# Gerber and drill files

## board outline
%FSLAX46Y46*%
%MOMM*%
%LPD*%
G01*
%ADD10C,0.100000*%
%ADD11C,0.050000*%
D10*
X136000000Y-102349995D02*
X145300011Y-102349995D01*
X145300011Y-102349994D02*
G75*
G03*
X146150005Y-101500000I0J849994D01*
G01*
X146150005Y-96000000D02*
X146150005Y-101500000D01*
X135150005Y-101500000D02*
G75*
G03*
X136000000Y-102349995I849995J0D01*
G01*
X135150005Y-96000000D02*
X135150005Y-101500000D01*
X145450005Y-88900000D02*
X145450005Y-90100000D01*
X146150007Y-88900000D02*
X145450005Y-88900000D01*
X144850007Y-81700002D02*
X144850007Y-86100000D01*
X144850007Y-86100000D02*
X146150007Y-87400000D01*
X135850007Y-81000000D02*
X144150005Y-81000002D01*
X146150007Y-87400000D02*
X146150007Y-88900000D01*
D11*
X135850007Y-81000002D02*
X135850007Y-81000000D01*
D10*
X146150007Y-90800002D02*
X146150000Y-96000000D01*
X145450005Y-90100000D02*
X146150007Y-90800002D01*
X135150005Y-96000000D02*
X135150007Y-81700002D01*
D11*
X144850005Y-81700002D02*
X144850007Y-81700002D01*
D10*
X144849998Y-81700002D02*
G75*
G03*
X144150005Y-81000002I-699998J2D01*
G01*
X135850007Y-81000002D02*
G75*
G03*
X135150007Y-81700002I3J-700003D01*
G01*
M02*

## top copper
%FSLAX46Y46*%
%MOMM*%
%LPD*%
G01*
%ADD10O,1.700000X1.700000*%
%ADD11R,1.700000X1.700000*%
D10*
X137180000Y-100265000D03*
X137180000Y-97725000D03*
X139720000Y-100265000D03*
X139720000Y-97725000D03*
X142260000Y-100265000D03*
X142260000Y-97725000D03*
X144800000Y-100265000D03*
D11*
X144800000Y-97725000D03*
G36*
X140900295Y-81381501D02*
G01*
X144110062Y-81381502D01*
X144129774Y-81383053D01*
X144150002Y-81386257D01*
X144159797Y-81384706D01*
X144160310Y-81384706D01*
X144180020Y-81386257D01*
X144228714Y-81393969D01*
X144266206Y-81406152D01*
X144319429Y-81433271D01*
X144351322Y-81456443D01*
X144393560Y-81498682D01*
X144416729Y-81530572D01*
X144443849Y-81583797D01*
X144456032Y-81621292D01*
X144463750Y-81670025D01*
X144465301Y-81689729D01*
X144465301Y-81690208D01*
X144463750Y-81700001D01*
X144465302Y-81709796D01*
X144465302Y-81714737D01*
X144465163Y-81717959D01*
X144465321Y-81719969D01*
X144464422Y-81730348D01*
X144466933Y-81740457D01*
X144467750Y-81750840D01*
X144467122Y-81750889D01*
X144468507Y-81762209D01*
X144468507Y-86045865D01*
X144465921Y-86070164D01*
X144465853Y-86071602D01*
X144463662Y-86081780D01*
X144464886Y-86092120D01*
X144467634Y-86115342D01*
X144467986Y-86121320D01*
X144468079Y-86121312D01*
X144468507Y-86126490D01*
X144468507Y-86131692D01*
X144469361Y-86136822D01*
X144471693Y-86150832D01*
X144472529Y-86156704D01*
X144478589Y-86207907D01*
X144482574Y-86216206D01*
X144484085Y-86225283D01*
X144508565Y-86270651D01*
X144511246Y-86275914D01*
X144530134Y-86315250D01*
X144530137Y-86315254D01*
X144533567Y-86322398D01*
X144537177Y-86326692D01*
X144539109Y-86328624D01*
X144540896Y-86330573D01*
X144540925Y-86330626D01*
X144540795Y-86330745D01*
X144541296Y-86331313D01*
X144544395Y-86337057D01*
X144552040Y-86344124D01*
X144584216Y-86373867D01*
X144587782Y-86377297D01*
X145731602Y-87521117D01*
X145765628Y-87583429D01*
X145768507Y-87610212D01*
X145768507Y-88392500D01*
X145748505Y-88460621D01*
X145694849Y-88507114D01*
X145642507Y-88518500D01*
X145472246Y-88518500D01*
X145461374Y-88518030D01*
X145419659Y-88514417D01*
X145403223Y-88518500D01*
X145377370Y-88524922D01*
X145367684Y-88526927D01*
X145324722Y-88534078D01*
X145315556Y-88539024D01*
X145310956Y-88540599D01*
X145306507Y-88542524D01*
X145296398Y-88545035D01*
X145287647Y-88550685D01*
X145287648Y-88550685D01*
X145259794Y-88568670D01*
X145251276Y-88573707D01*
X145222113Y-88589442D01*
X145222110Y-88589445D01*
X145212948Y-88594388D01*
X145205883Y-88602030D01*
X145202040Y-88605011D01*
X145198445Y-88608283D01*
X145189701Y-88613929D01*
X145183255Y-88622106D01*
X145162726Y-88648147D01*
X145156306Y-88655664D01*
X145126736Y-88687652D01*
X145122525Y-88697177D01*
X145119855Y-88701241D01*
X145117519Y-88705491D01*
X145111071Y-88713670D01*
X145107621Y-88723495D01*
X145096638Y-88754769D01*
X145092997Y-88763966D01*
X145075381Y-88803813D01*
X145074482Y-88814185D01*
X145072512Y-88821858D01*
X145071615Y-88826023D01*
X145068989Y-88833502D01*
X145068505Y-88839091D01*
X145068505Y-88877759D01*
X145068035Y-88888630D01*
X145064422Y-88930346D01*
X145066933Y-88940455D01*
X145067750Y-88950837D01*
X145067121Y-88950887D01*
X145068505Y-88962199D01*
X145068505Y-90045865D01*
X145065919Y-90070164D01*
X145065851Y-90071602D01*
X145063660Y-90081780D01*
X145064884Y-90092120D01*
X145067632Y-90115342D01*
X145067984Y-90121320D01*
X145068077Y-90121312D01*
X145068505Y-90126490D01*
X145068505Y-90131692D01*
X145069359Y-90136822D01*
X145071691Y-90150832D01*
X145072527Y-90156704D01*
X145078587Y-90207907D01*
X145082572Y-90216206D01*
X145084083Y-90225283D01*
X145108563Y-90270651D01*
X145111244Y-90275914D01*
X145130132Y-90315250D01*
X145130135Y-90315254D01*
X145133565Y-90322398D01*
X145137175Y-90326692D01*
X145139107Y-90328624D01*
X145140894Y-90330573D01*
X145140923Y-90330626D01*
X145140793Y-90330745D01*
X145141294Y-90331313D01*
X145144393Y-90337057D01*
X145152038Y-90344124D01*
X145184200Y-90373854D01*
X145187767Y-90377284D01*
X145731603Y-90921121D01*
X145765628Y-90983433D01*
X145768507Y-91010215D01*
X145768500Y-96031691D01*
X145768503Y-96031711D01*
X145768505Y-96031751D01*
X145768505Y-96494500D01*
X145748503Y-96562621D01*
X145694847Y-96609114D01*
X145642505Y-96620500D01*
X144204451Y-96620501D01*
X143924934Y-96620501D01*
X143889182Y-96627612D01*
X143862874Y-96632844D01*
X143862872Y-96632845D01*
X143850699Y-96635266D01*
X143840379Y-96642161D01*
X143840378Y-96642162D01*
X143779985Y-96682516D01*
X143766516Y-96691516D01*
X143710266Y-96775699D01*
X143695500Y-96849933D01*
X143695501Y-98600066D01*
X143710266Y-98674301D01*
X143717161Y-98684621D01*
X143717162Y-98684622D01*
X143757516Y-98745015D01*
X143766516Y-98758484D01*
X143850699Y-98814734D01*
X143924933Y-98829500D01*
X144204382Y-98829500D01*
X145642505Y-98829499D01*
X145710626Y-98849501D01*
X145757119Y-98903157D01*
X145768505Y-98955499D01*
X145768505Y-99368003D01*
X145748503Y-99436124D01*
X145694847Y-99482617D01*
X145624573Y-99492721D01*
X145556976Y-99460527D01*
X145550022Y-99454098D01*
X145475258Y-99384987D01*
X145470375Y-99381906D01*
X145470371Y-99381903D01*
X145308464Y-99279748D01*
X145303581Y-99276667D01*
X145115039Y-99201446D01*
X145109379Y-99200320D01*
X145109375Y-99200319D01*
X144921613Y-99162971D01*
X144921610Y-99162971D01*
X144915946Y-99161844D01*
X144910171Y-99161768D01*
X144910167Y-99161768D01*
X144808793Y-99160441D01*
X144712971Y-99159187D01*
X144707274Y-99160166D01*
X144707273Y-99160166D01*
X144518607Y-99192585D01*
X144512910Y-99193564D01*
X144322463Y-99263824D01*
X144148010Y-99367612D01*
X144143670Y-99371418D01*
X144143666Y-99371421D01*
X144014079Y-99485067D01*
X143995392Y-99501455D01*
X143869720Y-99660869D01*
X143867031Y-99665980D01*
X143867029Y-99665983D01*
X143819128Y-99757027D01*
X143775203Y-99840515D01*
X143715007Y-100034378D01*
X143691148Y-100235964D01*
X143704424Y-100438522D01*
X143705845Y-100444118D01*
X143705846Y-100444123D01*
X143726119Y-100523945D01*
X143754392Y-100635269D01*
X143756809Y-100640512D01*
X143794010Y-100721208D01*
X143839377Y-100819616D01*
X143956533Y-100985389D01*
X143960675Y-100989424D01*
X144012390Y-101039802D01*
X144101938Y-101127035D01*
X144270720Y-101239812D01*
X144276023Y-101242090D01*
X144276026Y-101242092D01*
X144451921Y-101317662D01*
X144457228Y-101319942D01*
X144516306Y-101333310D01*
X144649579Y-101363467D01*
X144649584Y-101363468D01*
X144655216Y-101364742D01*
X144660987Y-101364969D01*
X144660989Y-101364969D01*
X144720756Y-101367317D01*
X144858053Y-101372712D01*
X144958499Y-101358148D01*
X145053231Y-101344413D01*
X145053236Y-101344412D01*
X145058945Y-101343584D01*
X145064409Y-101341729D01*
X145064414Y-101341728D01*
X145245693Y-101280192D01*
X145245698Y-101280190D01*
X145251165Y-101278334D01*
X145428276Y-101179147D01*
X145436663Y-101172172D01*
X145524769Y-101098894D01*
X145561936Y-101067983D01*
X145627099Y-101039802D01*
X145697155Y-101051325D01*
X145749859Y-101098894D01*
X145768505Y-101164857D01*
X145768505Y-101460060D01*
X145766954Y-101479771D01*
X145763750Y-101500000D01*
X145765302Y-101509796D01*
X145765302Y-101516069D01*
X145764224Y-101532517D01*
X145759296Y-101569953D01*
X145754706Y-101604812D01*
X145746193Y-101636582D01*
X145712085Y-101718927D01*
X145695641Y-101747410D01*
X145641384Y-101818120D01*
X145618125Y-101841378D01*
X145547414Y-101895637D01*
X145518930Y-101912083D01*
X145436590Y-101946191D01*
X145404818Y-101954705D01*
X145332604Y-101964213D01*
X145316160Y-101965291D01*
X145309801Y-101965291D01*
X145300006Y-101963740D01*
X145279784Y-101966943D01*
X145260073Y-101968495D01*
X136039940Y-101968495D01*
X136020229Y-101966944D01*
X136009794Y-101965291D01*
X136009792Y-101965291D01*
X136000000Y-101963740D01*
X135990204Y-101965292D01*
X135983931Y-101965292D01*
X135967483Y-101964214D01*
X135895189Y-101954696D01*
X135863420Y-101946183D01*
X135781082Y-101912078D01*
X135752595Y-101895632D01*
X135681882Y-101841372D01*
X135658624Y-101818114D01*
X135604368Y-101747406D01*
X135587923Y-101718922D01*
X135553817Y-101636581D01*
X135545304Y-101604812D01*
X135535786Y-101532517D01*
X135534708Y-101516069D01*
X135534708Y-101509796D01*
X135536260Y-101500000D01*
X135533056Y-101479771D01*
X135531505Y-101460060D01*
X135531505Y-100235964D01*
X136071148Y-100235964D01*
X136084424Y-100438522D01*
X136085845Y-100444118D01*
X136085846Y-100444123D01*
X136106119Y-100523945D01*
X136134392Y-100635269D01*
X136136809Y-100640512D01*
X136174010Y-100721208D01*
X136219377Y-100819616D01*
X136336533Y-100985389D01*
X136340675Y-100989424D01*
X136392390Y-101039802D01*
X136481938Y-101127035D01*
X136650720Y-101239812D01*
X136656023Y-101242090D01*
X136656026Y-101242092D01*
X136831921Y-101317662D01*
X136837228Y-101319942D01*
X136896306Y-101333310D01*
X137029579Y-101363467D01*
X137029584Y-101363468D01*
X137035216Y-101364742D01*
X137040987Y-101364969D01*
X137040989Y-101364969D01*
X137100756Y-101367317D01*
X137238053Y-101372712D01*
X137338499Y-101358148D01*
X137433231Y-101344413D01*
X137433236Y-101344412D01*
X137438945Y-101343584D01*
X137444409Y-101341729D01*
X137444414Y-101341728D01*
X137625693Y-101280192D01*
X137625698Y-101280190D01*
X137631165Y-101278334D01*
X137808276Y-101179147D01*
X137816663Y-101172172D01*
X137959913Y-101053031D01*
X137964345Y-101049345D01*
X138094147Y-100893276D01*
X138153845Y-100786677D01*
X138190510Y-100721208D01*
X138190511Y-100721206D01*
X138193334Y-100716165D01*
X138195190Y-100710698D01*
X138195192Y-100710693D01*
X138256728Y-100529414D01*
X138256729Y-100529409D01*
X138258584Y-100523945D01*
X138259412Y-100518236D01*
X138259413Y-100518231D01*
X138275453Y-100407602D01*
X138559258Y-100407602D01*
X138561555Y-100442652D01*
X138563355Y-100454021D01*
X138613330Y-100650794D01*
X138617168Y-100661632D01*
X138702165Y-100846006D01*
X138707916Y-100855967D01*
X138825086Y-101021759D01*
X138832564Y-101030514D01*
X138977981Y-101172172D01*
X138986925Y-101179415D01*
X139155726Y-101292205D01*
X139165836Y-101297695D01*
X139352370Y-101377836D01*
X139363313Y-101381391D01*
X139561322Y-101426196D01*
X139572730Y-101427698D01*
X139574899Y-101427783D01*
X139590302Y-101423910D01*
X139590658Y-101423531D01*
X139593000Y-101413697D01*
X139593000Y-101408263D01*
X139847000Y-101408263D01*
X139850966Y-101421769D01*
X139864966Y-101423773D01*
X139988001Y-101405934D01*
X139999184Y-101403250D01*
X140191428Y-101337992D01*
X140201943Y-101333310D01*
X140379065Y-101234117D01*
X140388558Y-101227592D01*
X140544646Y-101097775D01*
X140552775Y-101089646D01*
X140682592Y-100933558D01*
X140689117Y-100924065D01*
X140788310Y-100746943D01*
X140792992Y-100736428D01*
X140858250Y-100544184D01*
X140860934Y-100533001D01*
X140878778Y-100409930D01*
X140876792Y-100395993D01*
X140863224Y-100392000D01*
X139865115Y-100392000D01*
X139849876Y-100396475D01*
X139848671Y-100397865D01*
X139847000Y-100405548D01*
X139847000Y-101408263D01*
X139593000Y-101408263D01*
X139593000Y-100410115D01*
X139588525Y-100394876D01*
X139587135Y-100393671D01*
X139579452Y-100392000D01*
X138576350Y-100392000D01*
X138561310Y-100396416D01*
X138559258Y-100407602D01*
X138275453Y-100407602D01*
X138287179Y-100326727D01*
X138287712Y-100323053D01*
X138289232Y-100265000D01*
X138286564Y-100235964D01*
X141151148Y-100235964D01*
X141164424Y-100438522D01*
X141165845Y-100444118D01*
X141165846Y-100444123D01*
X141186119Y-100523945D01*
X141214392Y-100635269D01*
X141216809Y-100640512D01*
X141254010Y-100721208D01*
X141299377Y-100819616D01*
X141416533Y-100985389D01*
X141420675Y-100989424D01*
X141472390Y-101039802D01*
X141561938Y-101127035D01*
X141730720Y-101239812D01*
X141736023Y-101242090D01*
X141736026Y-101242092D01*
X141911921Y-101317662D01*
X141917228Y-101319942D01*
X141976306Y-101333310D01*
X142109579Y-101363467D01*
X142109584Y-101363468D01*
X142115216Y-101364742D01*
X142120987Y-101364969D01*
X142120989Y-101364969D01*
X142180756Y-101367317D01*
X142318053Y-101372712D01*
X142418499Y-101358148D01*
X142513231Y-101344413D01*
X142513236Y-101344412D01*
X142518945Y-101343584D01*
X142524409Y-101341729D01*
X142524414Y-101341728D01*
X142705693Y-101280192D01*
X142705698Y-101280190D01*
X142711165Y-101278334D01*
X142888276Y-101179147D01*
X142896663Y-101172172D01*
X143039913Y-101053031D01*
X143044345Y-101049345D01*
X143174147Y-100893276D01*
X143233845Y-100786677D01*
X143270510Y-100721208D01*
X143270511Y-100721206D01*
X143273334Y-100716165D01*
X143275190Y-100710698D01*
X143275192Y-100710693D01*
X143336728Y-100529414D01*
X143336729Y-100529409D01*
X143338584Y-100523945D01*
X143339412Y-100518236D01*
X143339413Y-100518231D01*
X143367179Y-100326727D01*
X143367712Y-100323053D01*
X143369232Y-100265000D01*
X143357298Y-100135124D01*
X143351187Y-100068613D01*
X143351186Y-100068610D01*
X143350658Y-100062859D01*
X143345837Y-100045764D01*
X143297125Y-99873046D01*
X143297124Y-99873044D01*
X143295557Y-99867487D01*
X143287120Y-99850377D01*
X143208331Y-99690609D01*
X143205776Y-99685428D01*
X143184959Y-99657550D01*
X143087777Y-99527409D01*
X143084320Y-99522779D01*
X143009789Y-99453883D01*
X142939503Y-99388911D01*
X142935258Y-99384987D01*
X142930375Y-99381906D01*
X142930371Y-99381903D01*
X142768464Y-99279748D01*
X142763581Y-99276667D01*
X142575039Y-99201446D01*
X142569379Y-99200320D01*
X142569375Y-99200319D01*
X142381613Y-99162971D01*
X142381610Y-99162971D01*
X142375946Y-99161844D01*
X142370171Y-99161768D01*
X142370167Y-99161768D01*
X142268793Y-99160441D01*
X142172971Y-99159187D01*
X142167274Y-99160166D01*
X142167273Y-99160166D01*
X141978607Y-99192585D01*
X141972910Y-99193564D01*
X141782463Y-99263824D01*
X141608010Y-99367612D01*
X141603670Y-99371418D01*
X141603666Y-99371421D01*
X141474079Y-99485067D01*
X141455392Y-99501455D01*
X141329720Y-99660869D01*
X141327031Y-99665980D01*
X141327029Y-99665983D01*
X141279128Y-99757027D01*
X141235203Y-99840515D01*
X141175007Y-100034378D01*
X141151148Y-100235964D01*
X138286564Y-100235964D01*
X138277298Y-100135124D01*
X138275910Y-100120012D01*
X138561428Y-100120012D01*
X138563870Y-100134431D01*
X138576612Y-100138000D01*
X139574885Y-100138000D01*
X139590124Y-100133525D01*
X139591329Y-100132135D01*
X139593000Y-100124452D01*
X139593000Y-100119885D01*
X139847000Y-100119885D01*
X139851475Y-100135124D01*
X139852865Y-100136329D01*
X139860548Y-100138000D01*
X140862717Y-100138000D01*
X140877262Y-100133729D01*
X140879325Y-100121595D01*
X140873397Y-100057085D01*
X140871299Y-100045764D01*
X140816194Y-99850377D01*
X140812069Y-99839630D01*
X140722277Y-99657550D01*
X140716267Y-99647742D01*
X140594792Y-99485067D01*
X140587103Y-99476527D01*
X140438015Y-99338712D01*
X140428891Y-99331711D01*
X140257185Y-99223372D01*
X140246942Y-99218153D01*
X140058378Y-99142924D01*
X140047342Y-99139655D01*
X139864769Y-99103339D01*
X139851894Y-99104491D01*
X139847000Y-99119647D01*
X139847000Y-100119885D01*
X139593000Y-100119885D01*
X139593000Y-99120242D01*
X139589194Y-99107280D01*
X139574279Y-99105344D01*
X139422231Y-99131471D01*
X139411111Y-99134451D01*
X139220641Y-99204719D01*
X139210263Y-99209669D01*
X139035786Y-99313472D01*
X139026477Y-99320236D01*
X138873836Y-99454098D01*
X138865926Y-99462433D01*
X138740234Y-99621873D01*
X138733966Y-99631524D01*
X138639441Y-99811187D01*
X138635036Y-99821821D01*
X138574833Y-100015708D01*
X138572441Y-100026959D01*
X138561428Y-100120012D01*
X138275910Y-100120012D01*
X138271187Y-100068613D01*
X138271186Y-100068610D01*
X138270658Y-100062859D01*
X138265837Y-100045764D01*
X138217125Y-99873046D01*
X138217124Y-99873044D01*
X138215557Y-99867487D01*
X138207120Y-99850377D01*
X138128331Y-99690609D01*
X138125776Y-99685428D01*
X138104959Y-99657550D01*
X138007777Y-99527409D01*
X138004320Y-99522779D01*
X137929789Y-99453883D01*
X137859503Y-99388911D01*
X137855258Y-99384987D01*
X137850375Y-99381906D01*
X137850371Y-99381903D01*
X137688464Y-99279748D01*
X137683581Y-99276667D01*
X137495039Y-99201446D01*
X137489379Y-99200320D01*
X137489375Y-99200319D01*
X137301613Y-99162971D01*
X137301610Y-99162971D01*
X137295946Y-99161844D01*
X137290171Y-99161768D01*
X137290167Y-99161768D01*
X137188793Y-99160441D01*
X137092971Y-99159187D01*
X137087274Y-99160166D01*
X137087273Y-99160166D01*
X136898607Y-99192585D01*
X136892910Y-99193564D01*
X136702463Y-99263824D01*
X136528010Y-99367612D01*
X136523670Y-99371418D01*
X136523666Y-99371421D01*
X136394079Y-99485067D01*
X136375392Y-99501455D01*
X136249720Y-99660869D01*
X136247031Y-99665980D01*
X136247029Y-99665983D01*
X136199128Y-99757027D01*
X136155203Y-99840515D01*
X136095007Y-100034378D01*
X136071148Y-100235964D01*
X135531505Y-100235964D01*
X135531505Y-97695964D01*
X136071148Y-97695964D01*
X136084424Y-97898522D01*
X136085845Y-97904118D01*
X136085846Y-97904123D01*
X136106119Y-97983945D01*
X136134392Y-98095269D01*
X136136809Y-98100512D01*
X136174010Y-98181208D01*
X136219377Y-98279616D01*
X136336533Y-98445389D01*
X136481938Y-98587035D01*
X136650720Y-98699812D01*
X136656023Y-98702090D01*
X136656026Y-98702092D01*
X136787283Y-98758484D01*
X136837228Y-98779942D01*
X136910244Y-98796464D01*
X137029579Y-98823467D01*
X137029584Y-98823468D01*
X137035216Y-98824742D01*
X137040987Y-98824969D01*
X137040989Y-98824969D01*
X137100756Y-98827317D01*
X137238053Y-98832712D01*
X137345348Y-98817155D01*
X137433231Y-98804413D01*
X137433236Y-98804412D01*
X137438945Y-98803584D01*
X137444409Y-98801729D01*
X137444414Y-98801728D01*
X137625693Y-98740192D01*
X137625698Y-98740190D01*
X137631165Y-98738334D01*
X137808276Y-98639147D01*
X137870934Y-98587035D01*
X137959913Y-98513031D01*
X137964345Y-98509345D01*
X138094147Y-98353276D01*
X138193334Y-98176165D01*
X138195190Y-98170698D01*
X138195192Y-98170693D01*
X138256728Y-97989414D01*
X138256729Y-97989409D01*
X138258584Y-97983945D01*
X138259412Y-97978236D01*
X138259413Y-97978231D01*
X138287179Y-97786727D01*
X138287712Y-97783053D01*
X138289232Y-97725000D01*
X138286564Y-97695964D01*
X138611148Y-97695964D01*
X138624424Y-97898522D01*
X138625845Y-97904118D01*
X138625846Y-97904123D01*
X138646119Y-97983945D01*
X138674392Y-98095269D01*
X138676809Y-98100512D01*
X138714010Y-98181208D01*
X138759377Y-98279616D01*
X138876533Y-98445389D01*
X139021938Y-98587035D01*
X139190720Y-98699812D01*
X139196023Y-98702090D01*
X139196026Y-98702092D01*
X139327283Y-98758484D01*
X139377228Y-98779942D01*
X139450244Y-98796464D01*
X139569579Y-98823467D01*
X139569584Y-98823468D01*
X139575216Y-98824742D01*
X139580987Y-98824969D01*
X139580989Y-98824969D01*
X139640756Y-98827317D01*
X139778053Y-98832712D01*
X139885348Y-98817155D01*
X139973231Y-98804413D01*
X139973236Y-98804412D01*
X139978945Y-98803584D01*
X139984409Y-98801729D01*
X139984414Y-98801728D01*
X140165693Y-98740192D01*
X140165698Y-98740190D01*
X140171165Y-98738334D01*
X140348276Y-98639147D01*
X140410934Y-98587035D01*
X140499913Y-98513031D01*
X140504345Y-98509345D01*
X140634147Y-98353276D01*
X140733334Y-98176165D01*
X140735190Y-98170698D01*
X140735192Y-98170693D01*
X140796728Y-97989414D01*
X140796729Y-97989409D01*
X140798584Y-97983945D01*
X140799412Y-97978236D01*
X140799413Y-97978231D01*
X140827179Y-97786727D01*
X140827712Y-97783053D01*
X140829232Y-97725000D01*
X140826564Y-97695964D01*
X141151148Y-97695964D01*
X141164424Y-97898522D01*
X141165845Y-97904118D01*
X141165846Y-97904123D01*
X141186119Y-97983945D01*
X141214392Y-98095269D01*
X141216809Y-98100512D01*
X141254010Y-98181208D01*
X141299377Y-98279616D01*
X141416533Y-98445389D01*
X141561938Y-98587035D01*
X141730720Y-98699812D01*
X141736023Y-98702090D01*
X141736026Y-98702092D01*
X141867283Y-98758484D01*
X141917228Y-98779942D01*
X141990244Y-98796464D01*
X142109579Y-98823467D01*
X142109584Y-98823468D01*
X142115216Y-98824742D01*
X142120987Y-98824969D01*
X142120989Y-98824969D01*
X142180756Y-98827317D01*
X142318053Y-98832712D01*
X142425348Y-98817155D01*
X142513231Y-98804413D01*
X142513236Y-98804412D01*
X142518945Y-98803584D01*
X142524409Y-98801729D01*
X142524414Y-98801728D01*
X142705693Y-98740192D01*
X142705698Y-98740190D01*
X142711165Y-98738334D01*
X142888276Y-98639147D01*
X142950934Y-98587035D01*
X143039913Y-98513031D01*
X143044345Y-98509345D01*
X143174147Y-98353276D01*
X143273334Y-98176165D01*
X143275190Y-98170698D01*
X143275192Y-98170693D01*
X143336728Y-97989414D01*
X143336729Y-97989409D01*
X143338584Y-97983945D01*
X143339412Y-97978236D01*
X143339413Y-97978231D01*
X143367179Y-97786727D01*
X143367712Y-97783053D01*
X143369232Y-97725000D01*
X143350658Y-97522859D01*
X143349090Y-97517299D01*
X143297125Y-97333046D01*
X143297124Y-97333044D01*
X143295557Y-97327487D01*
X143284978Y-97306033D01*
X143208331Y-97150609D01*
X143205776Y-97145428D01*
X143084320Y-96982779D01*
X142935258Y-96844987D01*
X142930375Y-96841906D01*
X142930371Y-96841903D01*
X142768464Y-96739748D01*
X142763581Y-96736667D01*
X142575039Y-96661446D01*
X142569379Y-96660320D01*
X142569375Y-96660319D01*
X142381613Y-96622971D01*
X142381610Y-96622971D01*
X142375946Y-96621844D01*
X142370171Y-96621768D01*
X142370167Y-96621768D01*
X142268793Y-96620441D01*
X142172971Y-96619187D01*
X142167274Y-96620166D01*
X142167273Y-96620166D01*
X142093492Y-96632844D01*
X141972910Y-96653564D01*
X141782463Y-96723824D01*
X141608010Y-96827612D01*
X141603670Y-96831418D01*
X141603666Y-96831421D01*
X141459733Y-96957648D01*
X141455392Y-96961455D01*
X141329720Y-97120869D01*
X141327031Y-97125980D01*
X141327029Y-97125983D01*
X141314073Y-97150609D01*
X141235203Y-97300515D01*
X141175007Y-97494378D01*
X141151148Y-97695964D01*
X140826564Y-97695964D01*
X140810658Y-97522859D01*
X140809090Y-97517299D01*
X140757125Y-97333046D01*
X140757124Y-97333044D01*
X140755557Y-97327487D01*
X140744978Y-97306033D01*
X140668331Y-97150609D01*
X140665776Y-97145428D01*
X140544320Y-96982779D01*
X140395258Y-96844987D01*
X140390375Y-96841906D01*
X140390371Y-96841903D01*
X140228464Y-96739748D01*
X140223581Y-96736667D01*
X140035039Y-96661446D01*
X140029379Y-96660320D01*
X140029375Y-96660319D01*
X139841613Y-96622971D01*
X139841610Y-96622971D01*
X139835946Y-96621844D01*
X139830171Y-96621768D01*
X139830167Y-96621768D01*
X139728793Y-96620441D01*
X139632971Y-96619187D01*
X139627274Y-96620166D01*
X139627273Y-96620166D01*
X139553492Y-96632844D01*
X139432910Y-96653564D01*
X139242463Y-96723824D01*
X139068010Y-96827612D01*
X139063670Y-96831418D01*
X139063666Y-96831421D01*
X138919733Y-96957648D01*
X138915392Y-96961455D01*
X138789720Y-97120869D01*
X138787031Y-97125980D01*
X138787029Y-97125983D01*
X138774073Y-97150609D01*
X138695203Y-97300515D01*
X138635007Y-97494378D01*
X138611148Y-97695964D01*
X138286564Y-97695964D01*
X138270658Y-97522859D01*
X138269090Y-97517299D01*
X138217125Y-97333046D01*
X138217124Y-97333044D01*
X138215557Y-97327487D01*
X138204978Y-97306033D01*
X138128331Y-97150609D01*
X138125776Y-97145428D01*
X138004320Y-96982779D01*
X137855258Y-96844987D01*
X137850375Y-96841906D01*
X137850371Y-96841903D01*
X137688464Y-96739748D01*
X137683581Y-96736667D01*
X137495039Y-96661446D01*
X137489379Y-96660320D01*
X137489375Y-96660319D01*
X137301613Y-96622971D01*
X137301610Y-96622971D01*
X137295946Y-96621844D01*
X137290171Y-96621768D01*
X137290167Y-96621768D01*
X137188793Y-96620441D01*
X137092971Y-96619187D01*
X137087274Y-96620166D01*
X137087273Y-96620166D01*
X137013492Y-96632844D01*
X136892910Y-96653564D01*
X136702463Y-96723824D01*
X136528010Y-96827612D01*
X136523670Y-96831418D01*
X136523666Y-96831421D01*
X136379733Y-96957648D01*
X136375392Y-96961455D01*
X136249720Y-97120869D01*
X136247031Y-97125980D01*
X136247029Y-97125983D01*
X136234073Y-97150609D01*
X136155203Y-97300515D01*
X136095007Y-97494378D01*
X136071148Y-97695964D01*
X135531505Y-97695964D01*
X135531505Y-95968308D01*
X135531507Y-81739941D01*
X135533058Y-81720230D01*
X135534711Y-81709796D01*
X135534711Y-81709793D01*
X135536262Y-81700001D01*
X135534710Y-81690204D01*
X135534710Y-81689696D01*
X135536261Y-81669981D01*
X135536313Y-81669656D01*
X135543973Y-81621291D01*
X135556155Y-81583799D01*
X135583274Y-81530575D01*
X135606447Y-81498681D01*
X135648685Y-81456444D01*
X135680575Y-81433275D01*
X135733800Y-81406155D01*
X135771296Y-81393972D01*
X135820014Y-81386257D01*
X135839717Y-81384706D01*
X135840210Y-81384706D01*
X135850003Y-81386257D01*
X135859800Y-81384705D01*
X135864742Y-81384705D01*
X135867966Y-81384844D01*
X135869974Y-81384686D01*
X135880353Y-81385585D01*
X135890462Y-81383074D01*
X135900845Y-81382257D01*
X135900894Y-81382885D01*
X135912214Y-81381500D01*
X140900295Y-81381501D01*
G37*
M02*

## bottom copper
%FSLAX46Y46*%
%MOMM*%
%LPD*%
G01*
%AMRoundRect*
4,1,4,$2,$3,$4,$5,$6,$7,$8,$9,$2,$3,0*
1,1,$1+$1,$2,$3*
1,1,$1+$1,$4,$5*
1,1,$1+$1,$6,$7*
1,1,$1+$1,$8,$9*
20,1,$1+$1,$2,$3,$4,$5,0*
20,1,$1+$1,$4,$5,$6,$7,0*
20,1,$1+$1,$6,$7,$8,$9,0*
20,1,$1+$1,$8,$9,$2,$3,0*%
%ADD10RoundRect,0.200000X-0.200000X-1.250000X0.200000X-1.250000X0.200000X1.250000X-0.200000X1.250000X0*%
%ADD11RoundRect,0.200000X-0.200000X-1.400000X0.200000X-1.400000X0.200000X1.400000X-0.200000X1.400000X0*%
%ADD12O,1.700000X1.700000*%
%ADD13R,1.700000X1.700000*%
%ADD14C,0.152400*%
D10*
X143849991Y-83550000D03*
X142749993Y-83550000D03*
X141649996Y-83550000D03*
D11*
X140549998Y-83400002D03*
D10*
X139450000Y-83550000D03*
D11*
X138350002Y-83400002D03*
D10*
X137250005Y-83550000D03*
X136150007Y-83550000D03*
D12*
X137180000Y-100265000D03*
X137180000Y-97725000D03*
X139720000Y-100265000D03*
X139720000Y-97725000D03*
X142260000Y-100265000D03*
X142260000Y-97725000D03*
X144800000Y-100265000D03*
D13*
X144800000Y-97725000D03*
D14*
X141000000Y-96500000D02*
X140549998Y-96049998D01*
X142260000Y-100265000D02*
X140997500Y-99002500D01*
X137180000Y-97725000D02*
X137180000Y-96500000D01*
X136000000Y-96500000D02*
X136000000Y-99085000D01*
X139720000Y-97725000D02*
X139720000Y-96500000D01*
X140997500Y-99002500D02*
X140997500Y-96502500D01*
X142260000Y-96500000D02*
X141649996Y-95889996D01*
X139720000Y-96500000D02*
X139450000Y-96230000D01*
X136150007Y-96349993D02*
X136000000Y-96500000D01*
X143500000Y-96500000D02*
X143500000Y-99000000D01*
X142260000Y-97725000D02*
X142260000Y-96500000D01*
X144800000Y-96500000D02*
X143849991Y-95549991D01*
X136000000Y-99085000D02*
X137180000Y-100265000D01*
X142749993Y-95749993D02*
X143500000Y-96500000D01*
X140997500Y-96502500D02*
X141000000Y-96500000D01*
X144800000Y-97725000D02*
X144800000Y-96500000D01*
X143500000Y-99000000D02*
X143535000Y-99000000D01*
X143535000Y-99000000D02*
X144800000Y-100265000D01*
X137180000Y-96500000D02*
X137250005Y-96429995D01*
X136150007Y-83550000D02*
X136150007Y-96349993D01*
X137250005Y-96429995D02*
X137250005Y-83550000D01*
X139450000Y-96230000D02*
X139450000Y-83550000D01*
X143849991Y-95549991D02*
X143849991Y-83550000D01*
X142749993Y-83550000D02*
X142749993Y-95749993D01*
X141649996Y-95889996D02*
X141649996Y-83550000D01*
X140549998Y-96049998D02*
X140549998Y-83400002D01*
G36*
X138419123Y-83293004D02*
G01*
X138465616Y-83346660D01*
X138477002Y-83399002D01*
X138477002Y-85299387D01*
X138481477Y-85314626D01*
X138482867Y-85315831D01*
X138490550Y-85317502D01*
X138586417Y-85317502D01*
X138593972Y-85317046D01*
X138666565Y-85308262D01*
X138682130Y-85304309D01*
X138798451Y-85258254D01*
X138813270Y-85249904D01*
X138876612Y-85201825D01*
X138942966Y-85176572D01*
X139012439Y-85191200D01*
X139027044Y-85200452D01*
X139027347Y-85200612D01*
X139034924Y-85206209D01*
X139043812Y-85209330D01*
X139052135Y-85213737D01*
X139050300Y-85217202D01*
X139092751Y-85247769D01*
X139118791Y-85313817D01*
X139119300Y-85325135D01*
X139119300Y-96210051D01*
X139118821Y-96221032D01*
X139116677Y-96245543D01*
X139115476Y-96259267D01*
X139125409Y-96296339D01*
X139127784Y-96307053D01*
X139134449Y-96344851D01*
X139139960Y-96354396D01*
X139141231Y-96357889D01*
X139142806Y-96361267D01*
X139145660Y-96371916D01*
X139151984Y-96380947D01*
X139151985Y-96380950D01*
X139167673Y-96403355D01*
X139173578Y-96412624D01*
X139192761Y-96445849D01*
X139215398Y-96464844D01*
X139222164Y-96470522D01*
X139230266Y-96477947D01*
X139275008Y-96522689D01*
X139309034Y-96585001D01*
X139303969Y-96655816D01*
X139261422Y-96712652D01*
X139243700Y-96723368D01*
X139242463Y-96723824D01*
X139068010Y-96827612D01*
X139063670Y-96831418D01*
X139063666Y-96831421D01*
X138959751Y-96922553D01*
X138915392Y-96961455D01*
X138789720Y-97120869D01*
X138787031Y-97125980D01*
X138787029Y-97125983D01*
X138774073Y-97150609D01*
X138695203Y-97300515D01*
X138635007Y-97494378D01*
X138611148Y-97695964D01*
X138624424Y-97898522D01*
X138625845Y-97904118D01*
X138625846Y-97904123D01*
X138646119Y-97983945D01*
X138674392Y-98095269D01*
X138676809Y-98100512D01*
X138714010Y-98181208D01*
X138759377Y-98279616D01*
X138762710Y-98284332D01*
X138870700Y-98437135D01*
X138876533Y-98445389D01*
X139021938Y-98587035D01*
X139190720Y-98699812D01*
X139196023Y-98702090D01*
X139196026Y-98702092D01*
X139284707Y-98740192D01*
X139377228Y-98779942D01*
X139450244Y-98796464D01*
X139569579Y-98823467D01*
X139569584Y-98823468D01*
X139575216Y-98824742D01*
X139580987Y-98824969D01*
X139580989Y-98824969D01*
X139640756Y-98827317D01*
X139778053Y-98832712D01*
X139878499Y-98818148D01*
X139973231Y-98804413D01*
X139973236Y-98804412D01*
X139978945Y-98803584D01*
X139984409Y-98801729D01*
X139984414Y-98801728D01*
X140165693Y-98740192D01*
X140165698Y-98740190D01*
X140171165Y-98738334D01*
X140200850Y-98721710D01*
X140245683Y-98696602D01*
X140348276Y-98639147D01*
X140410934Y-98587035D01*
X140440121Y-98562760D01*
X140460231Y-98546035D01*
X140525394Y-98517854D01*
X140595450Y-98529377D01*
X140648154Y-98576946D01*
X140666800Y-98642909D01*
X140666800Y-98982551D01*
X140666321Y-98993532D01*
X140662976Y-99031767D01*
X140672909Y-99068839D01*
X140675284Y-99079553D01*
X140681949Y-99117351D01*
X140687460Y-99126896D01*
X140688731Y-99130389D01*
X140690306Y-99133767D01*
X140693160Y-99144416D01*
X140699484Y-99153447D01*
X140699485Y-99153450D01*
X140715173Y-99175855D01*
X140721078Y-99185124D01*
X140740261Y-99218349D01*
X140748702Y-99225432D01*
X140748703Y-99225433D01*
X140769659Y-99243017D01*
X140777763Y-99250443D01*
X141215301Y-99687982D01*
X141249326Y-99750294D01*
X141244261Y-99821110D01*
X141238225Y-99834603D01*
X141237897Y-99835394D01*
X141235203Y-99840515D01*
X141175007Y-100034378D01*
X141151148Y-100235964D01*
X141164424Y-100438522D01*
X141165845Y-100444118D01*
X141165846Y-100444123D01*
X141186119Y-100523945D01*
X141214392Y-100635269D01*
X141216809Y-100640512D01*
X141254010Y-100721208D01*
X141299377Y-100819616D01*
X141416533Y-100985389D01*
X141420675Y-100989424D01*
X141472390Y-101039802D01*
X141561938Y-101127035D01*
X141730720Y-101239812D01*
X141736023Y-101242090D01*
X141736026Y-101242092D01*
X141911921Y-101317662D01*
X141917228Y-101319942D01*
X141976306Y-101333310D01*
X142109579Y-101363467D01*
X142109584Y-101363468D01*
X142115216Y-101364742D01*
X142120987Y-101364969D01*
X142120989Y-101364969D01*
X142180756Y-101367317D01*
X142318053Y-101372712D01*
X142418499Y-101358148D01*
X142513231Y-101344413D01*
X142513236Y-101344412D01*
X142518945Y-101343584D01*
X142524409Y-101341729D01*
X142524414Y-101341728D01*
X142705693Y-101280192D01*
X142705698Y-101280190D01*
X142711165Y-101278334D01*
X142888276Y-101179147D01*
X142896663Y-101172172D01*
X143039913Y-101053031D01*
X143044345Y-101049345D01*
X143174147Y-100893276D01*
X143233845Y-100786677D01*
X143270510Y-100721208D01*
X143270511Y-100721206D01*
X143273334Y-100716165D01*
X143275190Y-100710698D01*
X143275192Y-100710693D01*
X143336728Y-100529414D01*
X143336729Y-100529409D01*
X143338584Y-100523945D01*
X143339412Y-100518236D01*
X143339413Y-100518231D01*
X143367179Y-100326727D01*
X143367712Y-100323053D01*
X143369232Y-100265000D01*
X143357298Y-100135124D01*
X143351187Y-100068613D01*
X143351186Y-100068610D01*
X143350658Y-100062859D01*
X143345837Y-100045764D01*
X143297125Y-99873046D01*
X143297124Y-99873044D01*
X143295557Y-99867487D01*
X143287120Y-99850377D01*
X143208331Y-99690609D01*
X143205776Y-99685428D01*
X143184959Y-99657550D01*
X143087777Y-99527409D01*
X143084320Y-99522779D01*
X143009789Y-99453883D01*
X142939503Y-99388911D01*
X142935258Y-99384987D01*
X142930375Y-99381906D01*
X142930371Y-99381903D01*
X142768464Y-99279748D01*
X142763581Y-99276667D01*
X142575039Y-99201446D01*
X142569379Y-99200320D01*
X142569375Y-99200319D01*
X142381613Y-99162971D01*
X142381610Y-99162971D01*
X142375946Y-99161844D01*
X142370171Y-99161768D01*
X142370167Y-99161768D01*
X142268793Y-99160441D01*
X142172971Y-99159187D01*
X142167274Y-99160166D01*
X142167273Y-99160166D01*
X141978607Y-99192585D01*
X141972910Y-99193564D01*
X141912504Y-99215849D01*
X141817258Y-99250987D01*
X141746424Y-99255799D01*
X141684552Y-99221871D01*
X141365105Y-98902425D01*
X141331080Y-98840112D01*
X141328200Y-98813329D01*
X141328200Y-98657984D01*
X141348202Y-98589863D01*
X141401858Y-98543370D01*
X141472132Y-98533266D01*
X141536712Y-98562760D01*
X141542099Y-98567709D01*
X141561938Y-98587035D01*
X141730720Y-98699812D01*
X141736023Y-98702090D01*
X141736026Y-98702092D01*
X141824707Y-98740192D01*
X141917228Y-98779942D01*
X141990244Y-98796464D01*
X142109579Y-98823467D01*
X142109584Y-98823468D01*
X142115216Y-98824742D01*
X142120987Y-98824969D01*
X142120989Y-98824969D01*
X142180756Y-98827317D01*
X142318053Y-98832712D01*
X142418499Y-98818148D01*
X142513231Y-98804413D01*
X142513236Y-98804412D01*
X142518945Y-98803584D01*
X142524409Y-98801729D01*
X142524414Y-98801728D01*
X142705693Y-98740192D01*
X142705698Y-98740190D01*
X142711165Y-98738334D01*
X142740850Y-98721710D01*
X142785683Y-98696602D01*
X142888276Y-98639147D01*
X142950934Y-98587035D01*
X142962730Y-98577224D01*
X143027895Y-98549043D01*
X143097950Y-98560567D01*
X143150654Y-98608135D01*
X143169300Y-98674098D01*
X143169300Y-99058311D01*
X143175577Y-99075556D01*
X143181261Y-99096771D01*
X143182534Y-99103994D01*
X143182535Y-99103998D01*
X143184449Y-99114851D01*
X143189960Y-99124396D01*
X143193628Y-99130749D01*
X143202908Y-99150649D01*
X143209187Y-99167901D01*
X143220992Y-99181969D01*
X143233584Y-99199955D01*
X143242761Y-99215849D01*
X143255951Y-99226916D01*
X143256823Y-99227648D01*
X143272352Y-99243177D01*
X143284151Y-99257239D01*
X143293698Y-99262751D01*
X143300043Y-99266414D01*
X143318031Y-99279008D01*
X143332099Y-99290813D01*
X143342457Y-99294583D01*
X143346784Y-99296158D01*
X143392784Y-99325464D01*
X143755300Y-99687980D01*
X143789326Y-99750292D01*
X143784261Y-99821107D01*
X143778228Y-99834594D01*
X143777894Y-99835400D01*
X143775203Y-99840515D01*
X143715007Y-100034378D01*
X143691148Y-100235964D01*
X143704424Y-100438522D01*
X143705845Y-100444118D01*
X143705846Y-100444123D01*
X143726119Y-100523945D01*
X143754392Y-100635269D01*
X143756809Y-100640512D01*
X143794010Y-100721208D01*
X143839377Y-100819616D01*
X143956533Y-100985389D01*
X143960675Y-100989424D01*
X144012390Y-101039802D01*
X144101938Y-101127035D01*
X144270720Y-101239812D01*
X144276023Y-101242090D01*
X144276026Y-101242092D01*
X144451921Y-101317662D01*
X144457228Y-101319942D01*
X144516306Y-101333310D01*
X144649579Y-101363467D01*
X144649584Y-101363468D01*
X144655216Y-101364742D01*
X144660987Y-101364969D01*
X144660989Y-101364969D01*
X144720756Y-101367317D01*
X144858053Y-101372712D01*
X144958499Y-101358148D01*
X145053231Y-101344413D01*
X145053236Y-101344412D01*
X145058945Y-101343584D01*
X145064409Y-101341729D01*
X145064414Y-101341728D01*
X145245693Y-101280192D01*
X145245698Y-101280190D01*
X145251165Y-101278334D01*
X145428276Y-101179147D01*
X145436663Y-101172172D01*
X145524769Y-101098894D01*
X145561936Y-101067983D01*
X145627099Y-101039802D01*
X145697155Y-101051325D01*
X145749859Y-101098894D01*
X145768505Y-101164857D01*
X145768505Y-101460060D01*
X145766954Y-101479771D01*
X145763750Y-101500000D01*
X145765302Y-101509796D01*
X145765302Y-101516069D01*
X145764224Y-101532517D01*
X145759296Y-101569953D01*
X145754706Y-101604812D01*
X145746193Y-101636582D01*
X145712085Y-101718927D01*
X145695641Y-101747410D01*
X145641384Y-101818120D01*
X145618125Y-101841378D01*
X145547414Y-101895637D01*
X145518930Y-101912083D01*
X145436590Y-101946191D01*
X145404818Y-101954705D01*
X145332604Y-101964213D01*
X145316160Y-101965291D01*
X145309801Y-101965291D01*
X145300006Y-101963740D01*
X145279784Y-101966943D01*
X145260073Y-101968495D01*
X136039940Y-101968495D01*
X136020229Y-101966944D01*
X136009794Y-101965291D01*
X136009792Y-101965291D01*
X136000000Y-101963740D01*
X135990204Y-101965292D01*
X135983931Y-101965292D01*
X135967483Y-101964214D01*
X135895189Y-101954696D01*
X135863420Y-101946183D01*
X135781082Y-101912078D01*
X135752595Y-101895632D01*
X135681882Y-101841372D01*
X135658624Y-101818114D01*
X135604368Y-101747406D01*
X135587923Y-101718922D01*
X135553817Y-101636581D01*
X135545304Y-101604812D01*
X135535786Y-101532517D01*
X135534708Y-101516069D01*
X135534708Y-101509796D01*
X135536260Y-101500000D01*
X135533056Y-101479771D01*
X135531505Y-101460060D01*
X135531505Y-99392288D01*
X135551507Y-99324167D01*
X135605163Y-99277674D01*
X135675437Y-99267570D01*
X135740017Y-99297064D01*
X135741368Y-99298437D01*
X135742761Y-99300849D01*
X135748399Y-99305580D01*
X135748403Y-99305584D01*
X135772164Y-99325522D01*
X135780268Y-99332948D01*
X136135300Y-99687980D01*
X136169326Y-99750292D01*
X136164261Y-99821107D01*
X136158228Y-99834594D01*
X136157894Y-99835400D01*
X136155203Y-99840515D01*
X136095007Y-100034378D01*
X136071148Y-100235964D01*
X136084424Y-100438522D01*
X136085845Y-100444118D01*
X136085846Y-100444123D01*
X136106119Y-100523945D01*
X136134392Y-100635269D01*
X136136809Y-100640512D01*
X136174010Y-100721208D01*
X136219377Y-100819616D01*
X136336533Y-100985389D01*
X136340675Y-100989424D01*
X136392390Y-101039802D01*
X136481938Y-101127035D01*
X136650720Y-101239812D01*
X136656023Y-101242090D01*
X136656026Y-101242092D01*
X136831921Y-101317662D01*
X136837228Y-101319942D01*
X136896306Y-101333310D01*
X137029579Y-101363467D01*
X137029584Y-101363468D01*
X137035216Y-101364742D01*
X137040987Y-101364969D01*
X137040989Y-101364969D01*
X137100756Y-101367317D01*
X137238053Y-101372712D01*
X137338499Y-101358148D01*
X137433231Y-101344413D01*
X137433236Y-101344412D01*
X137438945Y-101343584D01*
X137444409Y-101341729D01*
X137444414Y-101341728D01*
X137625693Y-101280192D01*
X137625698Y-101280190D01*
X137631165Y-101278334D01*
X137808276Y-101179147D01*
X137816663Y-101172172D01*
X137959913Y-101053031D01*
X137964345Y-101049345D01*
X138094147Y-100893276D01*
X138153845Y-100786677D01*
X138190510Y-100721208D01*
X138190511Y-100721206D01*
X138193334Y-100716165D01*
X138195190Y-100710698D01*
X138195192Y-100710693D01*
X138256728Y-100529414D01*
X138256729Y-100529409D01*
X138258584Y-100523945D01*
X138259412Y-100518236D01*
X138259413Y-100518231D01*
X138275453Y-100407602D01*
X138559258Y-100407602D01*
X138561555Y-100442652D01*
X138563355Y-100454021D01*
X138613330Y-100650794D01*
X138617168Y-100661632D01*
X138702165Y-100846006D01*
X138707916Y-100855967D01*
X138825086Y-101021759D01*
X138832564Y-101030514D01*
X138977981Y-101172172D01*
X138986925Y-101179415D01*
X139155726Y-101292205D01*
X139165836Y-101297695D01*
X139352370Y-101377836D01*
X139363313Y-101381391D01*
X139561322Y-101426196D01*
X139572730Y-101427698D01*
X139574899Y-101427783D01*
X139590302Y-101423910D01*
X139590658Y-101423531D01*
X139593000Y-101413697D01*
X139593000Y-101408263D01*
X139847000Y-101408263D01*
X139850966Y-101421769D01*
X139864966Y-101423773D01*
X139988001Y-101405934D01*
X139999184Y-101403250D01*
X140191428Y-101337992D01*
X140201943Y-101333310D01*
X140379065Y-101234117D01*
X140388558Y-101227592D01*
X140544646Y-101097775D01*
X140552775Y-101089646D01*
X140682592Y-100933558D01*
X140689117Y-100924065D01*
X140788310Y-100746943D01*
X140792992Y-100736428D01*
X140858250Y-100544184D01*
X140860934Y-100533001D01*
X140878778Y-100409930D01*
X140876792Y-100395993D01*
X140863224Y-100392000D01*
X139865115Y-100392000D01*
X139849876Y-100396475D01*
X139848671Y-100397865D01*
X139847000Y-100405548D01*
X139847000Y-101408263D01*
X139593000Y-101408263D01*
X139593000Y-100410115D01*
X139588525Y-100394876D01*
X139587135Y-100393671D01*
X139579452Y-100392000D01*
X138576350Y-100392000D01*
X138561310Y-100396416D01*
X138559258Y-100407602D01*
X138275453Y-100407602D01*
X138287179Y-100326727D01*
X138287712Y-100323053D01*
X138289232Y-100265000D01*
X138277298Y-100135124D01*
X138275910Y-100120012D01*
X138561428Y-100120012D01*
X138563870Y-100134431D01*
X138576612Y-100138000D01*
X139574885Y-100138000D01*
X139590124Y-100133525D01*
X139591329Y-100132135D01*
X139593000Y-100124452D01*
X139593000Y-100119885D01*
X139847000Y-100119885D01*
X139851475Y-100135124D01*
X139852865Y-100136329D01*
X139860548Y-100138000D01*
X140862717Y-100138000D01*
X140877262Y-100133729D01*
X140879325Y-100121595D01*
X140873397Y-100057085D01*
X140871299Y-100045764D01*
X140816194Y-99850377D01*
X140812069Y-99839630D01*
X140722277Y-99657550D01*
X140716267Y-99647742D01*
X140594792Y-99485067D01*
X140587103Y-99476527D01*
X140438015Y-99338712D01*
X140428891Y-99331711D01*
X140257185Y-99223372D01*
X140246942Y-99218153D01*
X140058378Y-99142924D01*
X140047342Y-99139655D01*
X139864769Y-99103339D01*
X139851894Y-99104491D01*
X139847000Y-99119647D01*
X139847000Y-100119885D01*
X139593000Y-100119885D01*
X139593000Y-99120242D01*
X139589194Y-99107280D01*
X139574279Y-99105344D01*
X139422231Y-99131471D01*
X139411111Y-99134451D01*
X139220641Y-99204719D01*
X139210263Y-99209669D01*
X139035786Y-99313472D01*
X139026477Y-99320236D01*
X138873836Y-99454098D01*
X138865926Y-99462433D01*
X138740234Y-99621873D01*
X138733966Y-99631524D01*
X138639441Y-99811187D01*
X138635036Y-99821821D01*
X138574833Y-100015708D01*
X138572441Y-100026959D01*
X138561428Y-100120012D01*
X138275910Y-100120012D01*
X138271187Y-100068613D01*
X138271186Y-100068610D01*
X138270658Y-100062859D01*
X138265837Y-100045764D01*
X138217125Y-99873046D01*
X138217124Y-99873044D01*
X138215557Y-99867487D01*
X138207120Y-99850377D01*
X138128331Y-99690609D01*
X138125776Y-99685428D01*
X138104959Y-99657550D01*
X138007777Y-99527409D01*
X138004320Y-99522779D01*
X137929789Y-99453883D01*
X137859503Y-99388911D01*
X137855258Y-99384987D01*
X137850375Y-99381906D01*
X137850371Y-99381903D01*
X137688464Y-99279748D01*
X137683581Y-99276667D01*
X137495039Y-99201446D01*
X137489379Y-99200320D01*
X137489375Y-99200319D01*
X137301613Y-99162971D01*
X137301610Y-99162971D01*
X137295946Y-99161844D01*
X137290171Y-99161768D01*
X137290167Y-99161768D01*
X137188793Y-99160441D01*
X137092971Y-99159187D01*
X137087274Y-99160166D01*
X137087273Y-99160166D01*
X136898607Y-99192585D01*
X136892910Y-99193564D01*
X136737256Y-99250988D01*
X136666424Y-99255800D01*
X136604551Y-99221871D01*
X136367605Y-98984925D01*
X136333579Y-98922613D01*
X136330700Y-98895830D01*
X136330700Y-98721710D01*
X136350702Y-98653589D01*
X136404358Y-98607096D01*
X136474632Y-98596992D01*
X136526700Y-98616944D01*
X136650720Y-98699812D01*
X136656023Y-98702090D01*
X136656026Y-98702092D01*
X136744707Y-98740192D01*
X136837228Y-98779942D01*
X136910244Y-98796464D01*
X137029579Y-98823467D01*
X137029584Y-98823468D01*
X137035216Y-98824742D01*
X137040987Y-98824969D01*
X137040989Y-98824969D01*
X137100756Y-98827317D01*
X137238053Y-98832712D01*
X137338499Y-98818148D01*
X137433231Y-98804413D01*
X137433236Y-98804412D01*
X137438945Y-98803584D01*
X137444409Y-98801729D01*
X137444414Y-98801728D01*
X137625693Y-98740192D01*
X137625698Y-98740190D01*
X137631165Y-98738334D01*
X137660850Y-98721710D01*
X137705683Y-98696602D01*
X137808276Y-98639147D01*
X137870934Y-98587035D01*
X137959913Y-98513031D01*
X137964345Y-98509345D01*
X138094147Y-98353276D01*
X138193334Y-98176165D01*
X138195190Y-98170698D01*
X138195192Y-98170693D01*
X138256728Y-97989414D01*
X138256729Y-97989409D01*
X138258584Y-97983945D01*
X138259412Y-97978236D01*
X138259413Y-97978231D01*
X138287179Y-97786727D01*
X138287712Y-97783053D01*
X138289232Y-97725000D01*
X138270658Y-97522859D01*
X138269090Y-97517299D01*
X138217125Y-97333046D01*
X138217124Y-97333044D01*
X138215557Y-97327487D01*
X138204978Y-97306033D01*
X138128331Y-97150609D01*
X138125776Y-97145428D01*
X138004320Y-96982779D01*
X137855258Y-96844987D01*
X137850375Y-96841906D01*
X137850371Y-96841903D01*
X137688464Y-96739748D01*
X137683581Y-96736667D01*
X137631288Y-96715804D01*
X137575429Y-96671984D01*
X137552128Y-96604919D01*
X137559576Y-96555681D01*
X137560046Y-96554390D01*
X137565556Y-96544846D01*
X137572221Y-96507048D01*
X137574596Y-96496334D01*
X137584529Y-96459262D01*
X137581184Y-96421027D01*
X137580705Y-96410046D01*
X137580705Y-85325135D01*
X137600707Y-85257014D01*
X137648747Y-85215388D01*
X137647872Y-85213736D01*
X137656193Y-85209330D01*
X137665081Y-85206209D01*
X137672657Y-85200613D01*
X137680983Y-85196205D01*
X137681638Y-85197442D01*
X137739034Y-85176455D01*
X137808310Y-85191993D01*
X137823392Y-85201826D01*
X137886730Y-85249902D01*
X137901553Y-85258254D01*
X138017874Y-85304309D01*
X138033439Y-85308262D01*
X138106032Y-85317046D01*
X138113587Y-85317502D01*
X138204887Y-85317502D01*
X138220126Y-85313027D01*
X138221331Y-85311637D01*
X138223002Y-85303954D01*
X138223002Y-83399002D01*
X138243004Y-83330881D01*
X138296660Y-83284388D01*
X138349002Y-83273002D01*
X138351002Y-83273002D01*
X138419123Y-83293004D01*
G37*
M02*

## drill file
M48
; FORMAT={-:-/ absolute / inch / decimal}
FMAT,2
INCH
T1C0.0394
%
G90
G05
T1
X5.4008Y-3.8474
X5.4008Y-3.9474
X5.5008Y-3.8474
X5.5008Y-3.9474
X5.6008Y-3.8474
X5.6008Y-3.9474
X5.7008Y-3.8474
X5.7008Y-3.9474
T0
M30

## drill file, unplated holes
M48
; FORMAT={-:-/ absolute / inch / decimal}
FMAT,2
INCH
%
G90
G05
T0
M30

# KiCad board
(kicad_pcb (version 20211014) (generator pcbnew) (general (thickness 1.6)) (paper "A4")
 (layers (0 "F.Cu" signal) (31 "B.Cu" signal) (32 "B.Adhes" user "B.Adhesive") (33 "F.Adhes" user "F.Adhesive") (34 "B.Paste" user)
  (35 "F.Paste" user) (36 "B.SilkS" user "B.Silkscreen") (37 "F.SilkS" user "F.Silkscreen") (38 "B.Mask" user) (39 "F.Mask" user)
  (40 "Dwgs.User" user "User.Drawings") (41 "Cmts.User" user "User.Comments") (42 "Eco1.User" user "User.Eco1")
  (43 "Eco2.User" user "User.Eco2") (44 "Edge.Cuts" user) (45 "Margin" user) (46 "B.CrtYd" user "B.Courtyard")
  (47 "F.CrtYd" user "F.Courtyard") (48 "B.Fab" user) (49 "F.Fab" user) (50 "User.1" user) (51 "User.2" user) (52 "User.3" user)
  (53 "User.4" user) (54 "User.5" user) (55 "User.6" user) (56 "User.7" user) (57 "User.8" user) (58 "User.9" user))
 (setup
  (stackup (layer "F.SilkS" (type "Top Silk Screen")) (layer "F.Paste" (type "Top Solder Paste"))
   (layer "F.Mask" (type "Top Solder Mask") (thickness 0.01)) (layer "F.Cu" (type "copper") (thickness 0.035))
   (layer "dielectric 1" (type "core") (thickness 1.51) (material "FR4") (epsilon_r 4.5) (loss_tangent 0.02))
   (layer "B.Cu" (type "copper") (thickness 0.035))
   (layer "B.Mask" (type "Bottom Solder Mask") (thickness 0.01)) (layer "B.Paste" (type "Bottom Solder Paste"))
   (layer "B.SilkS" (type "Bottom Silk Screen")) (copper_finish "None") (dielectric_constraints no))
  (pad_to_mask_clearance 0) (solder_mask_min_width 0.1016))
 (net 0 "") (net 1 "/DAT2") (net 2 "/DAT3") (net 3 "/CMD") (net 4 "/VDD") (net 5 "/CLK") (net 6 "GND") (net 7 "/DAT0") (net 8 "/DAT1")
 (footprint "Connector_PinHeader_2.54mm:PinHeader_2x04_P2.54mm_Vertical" (layer "F.Cu") (at 144.8 97.725 -90)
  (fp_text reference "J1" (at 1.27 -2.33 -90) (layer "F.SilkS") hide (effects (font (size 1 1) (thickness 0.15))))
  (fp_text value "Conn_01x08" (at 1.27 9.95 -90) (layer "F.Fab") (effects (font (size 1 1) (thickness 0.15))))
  (pad "1" thru_hole rect (at 0 0 270) (size 1.7 1.7) (drill 1) (layers *.Cu *.Mask) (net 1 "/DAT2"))
  (pad "2" thru_hole oval (at 2.54 0 270) (size 1.7 1.7) (drill 1) (layers *.Cu *.Mask) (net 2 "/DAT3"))
  (pad "3" thru_hole oval (at 0 2.54 270) (size 1.7 1.7) (drill 1) (layers *.Cu *.Mask) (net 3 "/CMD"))
  (pad "4" thru_hole oval (at 2.54 2.54 270) (size 1.7 1.7) (drill 1) (layers *.Cu *.Mask) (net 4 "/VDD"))
  (pad "5" thru_hole oval (at 0 5.08 270) (size 1.7 1.7) (drill 1) (layers *.Cu *.Mask) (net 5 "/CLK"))
  (pad "6" thru_hole oval (at 2.54 5.08 270) (size 1.7 1.7) (drill 1) (layers *.Cu *.Mask) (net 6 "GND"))
  (pad "7" thru_hole oval (at 0 7.62 270) (size 1.7 1.7) (drill 1) (layers *.Cu *.Mask) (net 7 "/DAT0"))
  (pad "8" thru_hole oval (at 2.54 7.62 270) (size 1.7 1.7) (drill 1) (layers *.Cu *.Mask) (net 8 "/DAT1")))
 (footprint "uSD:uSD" (layer "F.Cu") (at 140 90)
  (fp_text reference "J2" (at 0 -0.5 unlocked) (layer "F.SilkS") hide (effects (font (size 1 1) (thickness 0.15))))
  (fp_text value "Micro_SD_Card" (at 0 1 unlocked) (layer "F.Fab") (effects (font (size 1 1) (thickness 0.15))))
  (fp_line (start 4.850007 -8.299998) (end 4.850007 -3.9) (layer "Edge.Cuts") (width 0.1))
  (fp_line (start -4.149993 -9) (end 4.150005 -8.999998) (layer "Edge.Cuts") (width 0.1))
  (fp_line (start 4.850005 -8.299998) (end 4.850007 -8.299998) (layer "Edge.Cuts") (width 0.05))
  (fp_line (start 4.850007 -3.9) (end 6.150007 -2.6) (layer "Edge.Cuts") (width 0.1))
  (fp_line (start 6.150007 0.800002) (end 6.15 6) (layer "Edge.Cuts") (width 0.1))
  (fp_line (start 6.150007 -1.1) (end 5.450005 -1.1) (layer "Edge.Cuts") (width 0.1))
  (fp_line (start 5.450005 0.1) (end 6.150007 0.800002) (layer "Edge.Cuts") (width 0.1))
  (fp_line (start 6.150007 -2.6) (end 6.150007 -1.1) (layer "Edge.Cuts") (width 0.1))
  (fp_line (start -4.149993 -8.999998) (end -4.149993 -9) (layer "Edge.Cuts") (width 0.05))
  (fp_line (start -4.849995 6) (end -4.849993 -8.299998) (layer "Edge.Cuts") (width 0.1))
  (fp_line (start 5.450005 -1.1) (end 5.450005 0.1) (layer "Edge.Cuts") (width 0.1))
  (fp_arc (start -4.849993 -8.299998) (mid -4.644967 -8.794972) (end -4.149993 -8.999998) (layer "Edge.Cuts") (width 0.1))
  (fp_arc (start 4.150005 -8.999998) (mid 4.644976 -8.794971) (end 4.850005 -8.299998) (layer "Edge.Cuts") (width 0.1))
  (pad "1" smd roundrect (at 3.849991 -6.45) (size 0.8 2.9) (layers "B.Cu" "B.Paste" "B.Mask") (roundrect_rratio 0.25) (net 1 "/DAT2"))
  (pad "2" smd roundrect (at 2.749993 -6.45) (size 0.8 2.9) (layers "B.Cu" "B.Paste" "B.Mask") (roundrect_rratio 0.25) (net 2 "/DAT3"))
  (pad "3" smd roundrect (at 1.649996 -6.45) (size 0.8 2.9) (layers "B.Cu" "B.Paste" "B.Mask") (roundrect_rratio 0.25) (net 3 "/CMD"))
  (pad "4" smd roundrect (at 0.549998 -6.599998) (size 0.8 3.2) (layers "B.Cu" "B.Paste" "B.Mask") (roundrect_rratio 0.25) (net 4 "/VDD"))
  (pad "5" smd roundrect (at -0.55 -6.45) (size 0.8 2.9) (layers "B.Cu" "B.Paste" "B.Mask") (roundrect_rratio 0.25) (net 5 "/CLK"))
  (pad "6" smd roundrect (at -1.649998 -6.599998) (size 0.8 3.2) (layers "B.Cu" "B.Paste" "B.Mask") (roundrect_rratio 0.25) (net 6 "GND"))
  (pad "7" smd roundrect (at -2.749995 -6.45) (size 0.8 2.9) (layers "B.Cu" "B.Paste" "B.Mask") (roundrect_rratio 0.25) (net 7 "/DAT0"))
  (pad "8" smd roundrect (at -3.849993 -6.45) (size 0.8 2.9) (layers "B.Cu" "B.Paste" "B.Mask") (roundrect_rratio 0.25) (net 8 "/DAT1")))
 (gr_arc (start 136 102.349995) (mid 135.398963 102.101037) (end 135.150005 101.5) (layer "Edge.Cuts") (width 0.1))
 (gr_line (start 146.150005 96) (end 146.150005 101.5) (layer "Edge.Cuts") (width 0.1))
 (gr_line (start 135.150005 96) (end 135.150005 101.5) (layer "Edge.Cuts") (width 0.1))
 (gr_arc (start 146.150005 101.5) (mid 145.901048 102.101037) (end 145.300011 102.349995) (layer "Edge.Cuts") (width 0.1))
 (gr_line (start 136 102.349995) (end 145.300011 102.349995) (layer "Edge.Cuts") (width 0.1))
 (segment (start 143.849991 95.549991) (end 143.849991 83.55) (width 0.1524) (layer "B.Cu") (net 1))
 (segment (start 144.8 96.5) (end 143.849991 95.549991) (width 0.1524) (layer "B.Cu") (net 1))
 (segment (start 144.8 97.725) (end 144.8 96.5) (width 0.1524) (layer "B.Cu") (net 1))
 (segment (start 143.5 96.5) (end 143.5 99) (width 0.1524) (layer "B.Cu") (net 2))
 (segment (start 143.535 99) (end 144.8 100.265) (width 0.1524) (layer "B.Cu") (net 2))
 (segment (start 142.749993 95.749993) (end 143.5 96.5) (width 0.1524) (layer "B.Cu") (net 2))
 (segment (start 143.5 99) (end 143.535 99) (width 0.1524) (layer "B.Cu") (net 2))
 (segment (start 142.749993 83.55) (end 142.749993 95.749993) (width 0.1524) (layer "B.Cu") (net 2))
 (segment (start 141.649996 95.889996) (end 141.649996 83.55) (width 0.1524) (layer "B.Cu") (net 3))
 (segment (start 142.26 97.725) (end 142.26 96.5) (width 0.1524) (layer "B.Cu") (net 3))
 (segment (start 142.26 96.5) (end 141.649996 95.889996) (width 0.1524) (layer "B.Cu") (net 3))
 (segment (start 140.9975 99.0025) (end 140.9975 96.5025) (width 0.1524) (layer "B.Cu") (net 4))
 (segment (start 140.549998 96.049998) (end 140.549998 83.400002) (width 0.1524) (layer "B.Cu") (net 4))
 (segment (start 141 96.5) (end 140.549998 96.049998) (width 0.1524) (layer "B.Cu") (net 4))
 (segment (start 140.9975 96.5025) (end 141 96.5) (width 0.1524) (layer "B.Cu") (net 4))
 (segment (start 142.26 100.265) (end 140.9975 99.0025) (width 0.1524) (layer "B.Cu") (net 4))
 (segment (start 139.72 96.5) (end 139.45 96.23) (width 0.1524) (layer "B.Cu") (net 5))
 (segment (start 139.72 97.725) (end 139.72 96.5) (width 0.1524) (layer "B.Cu") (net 5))
 (segment (start 139.45 96.23) (end 139.45 83.55) (width 0.1524) (layer "B.Cu") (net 5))
 (segment (start 137.18 97.725) (end 137.18 96.5) (width 0.1524) (layer "B.Cu") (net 7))
 (segment (start 137.250005 96.429995) (end 137.250005 83.55) (width 0.1524) (layer "B.Cu") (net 7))
 (segment (start 137.18 96.5) (end 137.250005 96.429995) (width 0.1524) (layer "B.Cu") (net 7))
 (segment (start 136.150007 83.55) (end 136.150007 96.349993) (width 0.1524) (layer "B.Cu") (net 8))
 (segment (start 136 99.085) (end 137.18 100.265) (width 0.1524) (layer "B.Cu") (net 8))
 (segment (start 136 96.5) (end 136 99.085) (width 0.1524) (layer "B.Cu") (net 8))
 (segment (start 136.150007 96.349993) (end 136 96.5) (width 0.1524) (layer "B.Cu") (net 8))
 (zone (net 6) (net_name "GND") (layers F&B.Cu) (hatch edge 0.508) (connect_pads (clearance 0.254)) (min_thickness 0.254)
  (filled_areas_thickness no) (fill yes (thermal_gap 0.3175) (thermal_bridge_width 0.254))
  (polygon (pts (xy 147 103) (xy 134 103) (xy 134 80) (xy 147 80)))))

